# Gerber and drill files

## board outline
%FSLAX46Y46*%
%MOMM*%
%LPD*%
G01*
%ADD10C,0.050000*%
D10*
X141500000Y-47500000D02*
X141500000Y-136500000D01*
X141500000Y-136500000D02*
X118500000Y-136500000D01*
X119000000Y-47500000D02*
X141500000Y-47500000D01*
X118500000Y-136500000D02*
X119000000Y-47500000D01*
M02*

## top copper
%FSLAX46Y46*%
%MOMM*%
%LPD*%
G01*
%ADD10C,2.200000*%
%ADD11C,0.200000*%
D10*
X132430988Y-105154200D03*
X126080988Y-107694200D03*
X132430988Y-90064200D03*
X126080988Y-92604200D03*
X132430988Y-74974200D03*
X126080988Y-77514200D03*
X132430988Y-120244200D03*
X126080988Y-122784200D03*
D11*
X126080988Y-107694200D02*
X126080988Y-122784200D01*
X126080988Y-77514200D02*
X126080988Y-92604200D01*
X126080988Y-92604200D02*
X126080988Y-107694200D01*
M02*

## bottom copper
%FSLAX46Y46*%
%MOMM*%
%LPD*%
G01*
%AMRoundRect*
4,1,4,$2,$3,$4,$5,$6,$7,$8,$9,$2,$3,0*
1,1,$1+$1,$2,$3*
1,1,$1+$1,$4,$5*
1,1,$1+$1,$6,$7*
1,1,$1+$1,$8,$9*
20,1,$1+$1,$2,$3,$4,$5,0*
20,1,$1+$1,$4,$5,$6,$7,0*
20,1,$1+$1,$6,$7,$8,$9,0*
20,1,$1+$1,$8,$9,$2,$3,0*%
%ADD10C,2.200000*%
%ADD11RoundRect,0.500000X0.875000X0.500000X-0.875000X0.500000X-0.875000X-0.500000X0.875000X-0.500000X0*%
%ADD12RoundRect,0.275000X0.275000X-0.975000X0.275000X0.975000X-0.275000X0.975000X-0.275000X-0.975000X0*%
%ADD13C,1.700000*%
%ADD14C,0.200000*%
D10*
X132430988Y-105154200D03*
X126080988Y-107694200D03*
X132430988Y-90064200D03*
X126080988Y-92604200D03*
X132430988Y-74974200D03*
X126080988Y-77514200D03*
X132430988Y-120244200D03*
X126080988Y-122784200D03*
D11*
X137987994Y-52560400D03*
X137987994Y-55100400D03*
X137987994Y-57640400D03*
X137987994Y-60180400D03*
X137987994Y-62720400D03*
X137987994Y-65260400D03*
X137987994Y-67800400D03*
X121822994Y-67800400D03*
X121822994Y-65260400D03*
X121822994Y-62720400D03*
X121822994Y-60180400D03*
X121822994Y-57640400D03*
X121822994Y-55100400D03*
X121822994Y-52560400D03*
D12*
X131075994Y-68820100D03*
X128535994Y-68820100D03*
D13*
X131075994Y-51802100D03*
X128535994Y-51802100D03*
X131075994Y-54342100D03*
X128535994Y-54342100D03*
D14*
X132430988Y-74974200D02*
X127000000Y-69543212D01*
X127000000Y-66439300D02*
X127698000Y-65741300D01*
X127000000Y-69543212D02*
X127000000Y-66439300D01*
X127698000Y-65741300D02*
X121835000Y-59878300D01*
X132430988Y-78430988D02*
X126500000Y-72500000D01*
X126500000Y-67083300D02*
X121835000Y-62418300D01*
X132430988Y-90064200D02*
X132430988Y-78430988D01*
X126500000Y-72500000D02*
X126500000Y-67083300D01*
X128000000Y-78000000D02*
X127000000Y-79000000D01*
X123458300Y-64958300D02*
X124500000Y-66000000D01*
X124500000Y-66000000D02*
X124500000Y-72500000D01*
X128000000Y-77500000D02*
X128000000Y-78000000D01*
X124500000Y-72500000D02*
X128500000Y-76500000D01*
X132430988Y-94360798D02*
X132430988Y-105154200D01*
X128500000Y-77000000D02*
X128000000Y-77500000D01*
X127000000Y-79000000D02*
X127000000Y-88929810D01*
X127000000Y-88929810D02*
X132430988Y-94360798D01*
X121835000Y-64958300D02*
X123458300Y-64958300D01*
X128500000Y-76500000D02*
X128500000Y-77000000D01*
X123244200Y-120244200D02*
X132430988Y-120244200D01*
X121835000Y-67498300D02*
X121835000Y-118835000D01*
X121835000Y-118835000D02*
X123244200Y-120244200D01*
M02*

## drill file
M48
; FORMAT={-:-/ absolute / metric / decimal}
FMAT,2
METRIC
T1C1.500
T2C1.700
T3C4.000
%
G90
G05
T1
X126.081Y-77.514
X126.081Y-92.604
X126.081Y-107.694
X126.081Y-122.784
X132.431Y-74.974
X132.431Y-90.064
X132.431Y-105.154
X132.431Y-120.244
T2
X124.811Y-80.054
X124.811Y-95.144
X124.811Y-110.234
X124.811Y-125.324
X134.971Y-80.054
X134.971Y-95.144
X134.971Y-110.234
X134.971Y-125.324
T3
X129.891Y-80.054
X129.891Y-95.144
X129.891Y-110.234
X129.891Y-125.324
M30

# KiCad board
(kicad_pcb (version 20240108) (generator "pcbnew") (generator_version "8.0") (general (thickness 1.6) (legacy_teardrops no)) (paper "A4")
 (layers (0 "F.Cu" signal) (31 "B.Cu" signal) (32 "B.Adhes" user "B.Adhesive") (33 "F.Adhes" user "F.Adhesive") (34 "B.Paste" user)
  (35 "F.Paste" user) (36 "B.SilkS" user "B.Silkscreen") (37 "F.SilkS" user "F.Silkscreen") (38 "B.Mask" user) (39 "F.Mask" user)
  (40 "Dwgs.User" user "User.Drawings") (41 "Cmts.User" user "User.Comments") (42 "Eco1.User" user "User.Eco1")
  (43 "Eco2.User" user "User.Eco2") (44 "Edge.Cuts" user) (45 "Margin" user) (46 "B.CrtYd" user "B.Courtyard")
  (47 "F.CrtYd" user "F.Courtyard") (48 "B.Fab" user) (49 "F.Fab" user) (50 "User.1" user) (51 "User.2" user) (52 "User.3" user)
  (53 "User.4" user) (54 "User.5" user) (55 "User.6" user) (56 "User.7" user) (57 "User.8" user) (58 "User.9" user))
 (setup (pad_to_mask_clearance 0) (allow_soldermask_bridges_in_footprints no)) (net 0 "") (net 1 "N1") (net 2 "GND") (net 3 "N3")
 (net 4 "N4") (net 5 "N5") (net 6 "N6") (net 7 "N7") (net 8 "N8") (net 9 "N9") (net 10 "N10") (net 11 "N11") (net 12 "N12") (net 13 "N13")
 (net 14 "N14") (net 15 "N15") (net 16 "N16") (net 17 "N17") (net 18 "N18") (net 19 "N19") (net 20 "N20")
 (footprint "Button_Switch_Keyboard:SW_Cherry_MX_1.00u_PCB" (layer "F.Cu") (at 132.430988 105.1542)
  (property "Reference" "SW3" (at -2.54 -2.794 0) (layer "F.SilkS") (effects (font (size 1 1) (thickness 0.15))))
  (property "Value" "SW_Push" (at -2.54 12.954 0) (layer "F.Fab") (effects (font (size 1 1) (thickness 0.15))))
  (pad "" np_thru_hole circle (at -7.62 5.08) (size 1.7 1.7) (drill 1.7) (layers "*.Cu" "*.Mask"))
  (pad "" np_thru_hole circle (at -2.54 5.08) (size 4 4) (drill 4) (layers "*.Cu" "*.Mask"))
  (pad "" np_thru_hole circle (at 2.54 5.08) (size 1.7 1.7) (drill 1.7) (layers "*.Cu" "*.Mask"))
  (pad "1" thru_hole circle (at 0 0) (size 2.2 2.2) (drill 1.5) (layers "*.Cu" "*.Mask") (remove_unused_layers no) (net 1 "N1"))
  (pad "2" thru_hole circle (at -6.35 2.54) (size 2.2 2.2) (drill 1.5) (layers "*.Cu" "*.Mask") (remove_unused_layers no) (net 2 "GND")))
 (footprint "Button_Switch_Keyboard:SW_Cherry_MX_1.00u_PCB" (layer "F.Cu") (at 132.430988 90.0642)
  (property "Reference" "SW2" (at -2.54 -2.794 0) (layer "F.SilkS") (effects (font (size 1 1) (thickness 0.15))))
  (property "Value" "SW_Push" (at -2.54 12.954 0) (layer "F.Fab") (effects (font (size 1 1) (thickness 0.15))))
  (pad "" np_thru_hole circle (at -7.62 5.08) (size 1.7 1.7) (drill 1.7) (layers "*.Cu" "*.Mask"))
  (pad "" np_thru_hole circle (at -2.54 5.08) (size 4 4) (drill 4) (layers "*.Cu" "*.Mask"))
  (pad "" np_thru_hole circle (at 2.54 5.08) (size 1.7 1.7) (drill 1.7) (layers "*.Cu" "*.Mask"))
  (pad "1" thru_hole circle (at 0 0) (size 2.2 2.2) (drill 1.5) (layers "*.Cu" "*.Mask") (remove_unused_layers no) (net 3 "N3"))
  (pad "2" thru_hole circle (at -6.35 2.54) (size 2.2 2.2) (drill 1.5) (layers "*.Cu" "*.Mask") (remove_unused_layers no) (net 2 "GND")))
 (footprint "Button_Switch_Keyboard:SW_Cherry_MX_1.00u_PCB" (layer "F.Cu") (at 132.430988 74.9742)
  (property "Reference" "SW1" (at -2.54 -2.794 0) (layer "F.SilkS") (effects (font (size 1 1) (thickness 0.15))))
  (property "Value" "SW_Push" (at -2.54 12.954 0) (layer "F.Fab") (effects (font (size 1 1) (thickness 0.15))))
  (pad "" np_thru_hole circle (at -7.62 5.08) (size 1.7 1.7) (drill 1.7) (layers "*.Cu" "*.Mask"))
  (pad "" np_thru_hole circle (at -2.54 5.08) (size 4 4) (drill 4) (layers "*.Cu" "*.Mask"))
  (pad "" np_thru_hole circle (at 2.54 5.08) (size 1.7 1.7) (drill 1.7) (layers "*.Cu" "*.Mask"))
  (pad "1" thru_hole circle (at 0 0) (size 2.2 2.2) (drill 1.5) (layers "*.Cu" "*.Mask") (remove_unused_layers no) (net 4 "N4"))
  (pad "2" thru_hole circle (at -6.35 2.54) (size 2.2 2.2) (drill 1.5) (layers "*.Cu" "*.Mask") (remove_unused_layers no) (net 2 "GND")))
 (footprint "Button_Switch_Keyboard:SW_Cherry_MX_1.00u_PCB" (layer "F.Cu") (at 132.430988 120.2442)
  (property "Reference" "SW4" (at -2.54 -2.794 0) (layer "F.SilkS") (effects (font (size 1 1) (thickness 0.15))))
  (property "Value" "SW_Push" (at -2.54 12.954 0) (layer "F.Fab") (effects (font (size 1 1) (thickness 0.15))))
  (pad "" np_thru_hole circle (at -7.62 5.08) (size 1.7 1.7) (drill 1.7) (layers "*.Cu" "*.Mask"))
  (pad "" np_thru_hole circle (at -2.54 5.08) (size 4 4) (drill 4) (layers "*.Cu" "*.Mask"))
  (pad "" np_thru_hole circle (at 2.54 5.08) (size 1.7 1.7) (drill 1.7) (layers "*.Cu" "*.Mask"))
  (pad "1" thru_hole circle (at 0 0) (size 2.2 2.2) (drill 1.5) (layers "*.Cu" "*.Mask") (remove_unused_layers no) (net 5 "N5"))
  (pad "2" thru_hole circle (at -6.35 2.54) (size 2.2 2.2) (drill 1.5) (layers "*.Cu" "*.Mask") (remove_unused_layers no) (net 2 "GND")))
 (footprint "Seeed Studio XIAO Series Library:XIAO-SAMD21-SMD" (layer "B.Cu") (at 138.822994 70.6804 180)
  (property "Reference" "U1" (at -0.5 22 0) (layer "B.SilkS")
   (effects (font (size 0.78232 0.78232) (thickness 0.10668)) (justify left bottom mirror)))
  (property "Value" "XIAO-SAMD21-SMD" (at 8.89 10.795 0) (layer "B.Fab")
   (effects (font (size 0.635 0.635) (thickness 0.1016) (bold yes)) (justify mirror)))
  (pad "1" smd roundrect (at 0.835 18.12 180) (size 2.75 2) (layers "B.Cu" "B.Paste" "B.Mask") (roundrect_rratio 0.25) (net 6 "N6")
   (solder_mask_margin 0.0508) (thermal_bridge_angle 45))
  (pad "2" smd roundrect (at 0.835 15.58 180) (size 2.75 2) (layers "B.Cu" "B.Paste" "B.Mask") (roundrect_rratio 0.25) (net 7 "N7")
   (solder_mask_margin 0.0508) (thermal_bridge_angle 45))
  (pad "3" smd roundrect (at 0.835 13.04 180) (size 2.75 2) (layers "B.Cu" "B.Paste" "B.Mask") (roundrect_rratio 0.25) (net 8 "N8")
   (solder_mask_margin 0.0508) (thermal_bridge_angle 45))
  (pad "4" smd roundrect (at 0.835 10.5 180) (size 2.75 2) (layers "B.Cu" "B.Paste" "B.Mask") (roundrect_rratio 0.25) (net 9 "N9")
   (solder_mask_margin 0.0508) (thermal_bridge_angle 45))
  (pad "5" smd roundrect (at 0.835 7.96 180) (size 2.75 2) (layers "B.Cu" "B.Paste" "B.Mask") (roundrect_rratio 0.25) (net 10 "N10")
   (solder_mask_margin 0.0508) (thermal_bridge_angle 45))
  (pad "6" smd roundrect (at 0.835 5.42 180) (size 2.75 2) (layers "B.Cu" "B.Paste" "B.Mask") (roundrect_rratio 0.25) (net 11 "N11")
   (solder_mask_margin 0.0508) (thermal_bridge_angle 45))
  (pad "7" smd roundrect (at 0.835 2.88 180) (size 2.75 2) (layers "B.Cu" "B.Paste" "B.Mask") (roundrect_rratio 0.25) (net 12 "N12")
   (solder_mask_margin 0.0508) (thermal_bridge_angle 45))
  (pad "8" smd roundrect (at 17 2.88 180) (size 2.75 2) (layers "B.Cu" "B.Paste" "B.Mask") (roundrect_rratio 0.25) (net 5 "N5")
   (solder_mask_margin 0.0508) (thermal_bridge_angle 45))
  (pad "9" smd roundrect (at 17 5.42 180) (size 2.75 2) (layers "B.Cu" "B.Paste" "B.Mask") (roundrect_rratio 0.25) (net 1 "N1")
   (solder_mask_margin 0.0508) (thermal_bridge_angle 45))
  (pad "10" smd roundrect (at 17 7.96 180) (size 2.75 2) (layers "B.Cu" "B.Paste" "B.Mask") (roundrect_rratio 0.25) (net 3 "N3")
   (solder_mask_margin 0.0508) (thermal_bridge_angle 45))
  (pad "11" smd roundrect (at 17 10.5 180) (size 2.75 2) (layers "B.Cu" "B.Paste" "B.Mask") (roundrect_rratio 0.25) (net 4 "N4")
   (solder_mask_margin 0.0508) (thermal_bridge_angle 45))
  (pad "12" smd roundrect (at 17 13.04 180) (size 2.75 2) (layers "B.Cu" "B.Paste" "B.Mask") (roundrect_rratio 0.25) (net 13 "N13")
   (solder_mask_margin 0.0508) (thermal_bridge_angle 45))
  (pad "13" smd roundrect (at 17 15.58 180) (size 2.75 2) (layers "B.Cu" "B.Paste" "B.Mask") (roundrect_rratio 0.25) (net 2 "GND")
   (solder_mask_margin 0.0508) (thermal_bridge_angle 45))
  (pad "14" smd roundrect (at 17 18.12 180) (size 2.75 2) (layers "B.Cu" "B.Paste" "B.Mask") (roundrect_rratio 0.25) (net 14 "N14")
   (solder_mask_margin 0.0508) (thermal_bridge_angle 45))
  (pad "15" smd roundrect (at 7.747 1.8603 90) (size 2.5 1.1) (layers "B.Cu" "B.Paste" "B.Mask") (roundrect_rratio 0.25) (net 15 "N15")
   (solder_mask_margin 0.0508) (thermal_bridge_angle 45))
  (pad "16" smd roundrect (at 10.287 1.8603 90) (size 2.5 1.1) (layers "B.Cu" "B.Paste" "B.Mask") (roundrect_rratio 0.25) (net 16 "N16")
   (solder_mask_margin 0.0508) (thermal_bridge_angle 45))
  (pad "17" smd circle (at 7.747 18.8783 180) (size 1.7 1.7) (layers "B.Cu" "B.Paste" "B.Mask") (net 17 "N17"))
  (pad "18" smd circle (at 10.287 18.8783 180) (size 1.7 1.7) (layers "B.Cu" "B.Paste" "B.Mask") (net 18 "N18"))
  (pad "19" smd circle (at 7.747 16.3383 180) (size 1.7 1.7) (layers "B.Cu" "B.Paste" "B.Mask") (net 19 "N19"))
  (pad "20" smd circle (at 10.287 16.3383 180) (size 1.7 1.7) (layers "B.Cu" "B.Paste" "B.Mask") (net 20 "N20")))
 (gr_line (start 141.5 47.5) (end 141.5 136.5) (stroke (width 0.05) (type default)) (layer "Edge.Cuts"))
 (gr_line (start 141.5 136.5) (end 118.5 136.5) (stroke (width 0.05) (type default)) (layer "Edge.Cuts"))
 (gr_line (start 119 47.5) (end 141.5 47.5) (stroke (width 0.05) (type default)) (layer "Edge.Cuts"))
 (gr_line (start 118.5 136.5) (end 119 47.5) (stroke (width 0.05) (type default)) (layer "Edge.Cuts"))
 (segment (start 126.080988 107.6942) (end 126.080988 122.7842) (width 0.2) (layer "F.Cu") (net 2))
 (segment (start 126.080988 77.5142) (end 126.080988 92.6042) (width 0.2) (layer "F.Cu") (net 2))
 (segment (start 126.080988 92.6042) (end 126.080988 107.6942) (width 0.2) (layer "F.Cu") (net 2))
 (segment (start 132.430988 74.9742) (end 127 69.543212) (width 0.2) (layer "B.Cu") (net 4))
 (segment (start 127 66.4393) (end 127.698 65.7413) (width 0.2) (layer "B.Cu") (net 4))
 (segment (start 127 69.543212) (end 127 66.4393) (width 0.2) (layer "B.Cu") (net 4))
 (segment (start 127.698 65.7413) (end 121.835 59.8783) (width 0.2) (layer "B.Cu") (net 4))
 (segment (start 132.430988 78.430988) (end 126.5 72.5) (width 0.2) (layer "B.Cu") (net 3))
 (segment (start 126.5 67.0833) (end 121.835 62.4183) (width 0.2) (layer "B.Cu") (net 3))
 (segment (start 132.430988 90.0642) (end 132.430988 78.430988) (width 0.2) (layer "B.Cu") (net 3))
 (segment (start 126.5 72.5) (end 126.5 67.0833) (width 0.2) (layer "B.Cu") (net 3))
 (segment (start 128 78) (end 127 79) (width 0.2) (layer "B.Cu") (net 1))
 (segment (start 123.4583 64.9583) (end 124.5 66) (width 0.2) (layer "B.Cu") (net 1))
 (segment (start 124.5 66) (end 124.5 72.5) (width 0.2) (layer "B.Cu") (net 1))
 (segment (start 128 77.5) (end 128 78) (width 0.2) (layer "B.Cu") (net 1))
 (segment (start 124.5 72.5) (end 128.5 76.5) (width 0.2) (layer "B.Cu") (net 1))
 (segment (start 132.430988 94.360798) (end 132.430988 105.1542) (width 0.2) (layer "B.Cu") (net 1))
 (segment (start 128.5 77) (end 128 77.5) (width 0.2) (layer "B.Cu") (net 1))
 (segment (start 127 79) (end 127 88.92981) (width 0.2) (layer "B.Cu") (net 1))
 (segment (start 127 88.92981) (end 132.430988 94.360798) (width 0.2) (layer "B.Cu") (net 1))
 (segment (start 121.835 64.9583) (end 123.4583 64.9583) (width 0.2) (layer "B.Cu") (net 1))
 (segment (start 128.5 76.5) (end 128.5 77) (width 0.2) (layer "B.Cu") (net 1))
 (segment (start 123.2442 120.2442) (end 132.430988 120.2442) (width 0.2) (layer "B.Cu") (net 5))
 (segment (start 121.835 67.4983) (end 121.835 118.835) (width 0.2) (layer "B.Cu") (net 5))
 (segment (start 121.835 118.835) (end 123.2442 120.2442) (width 0.2) (layer "B.Cu") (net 5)))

